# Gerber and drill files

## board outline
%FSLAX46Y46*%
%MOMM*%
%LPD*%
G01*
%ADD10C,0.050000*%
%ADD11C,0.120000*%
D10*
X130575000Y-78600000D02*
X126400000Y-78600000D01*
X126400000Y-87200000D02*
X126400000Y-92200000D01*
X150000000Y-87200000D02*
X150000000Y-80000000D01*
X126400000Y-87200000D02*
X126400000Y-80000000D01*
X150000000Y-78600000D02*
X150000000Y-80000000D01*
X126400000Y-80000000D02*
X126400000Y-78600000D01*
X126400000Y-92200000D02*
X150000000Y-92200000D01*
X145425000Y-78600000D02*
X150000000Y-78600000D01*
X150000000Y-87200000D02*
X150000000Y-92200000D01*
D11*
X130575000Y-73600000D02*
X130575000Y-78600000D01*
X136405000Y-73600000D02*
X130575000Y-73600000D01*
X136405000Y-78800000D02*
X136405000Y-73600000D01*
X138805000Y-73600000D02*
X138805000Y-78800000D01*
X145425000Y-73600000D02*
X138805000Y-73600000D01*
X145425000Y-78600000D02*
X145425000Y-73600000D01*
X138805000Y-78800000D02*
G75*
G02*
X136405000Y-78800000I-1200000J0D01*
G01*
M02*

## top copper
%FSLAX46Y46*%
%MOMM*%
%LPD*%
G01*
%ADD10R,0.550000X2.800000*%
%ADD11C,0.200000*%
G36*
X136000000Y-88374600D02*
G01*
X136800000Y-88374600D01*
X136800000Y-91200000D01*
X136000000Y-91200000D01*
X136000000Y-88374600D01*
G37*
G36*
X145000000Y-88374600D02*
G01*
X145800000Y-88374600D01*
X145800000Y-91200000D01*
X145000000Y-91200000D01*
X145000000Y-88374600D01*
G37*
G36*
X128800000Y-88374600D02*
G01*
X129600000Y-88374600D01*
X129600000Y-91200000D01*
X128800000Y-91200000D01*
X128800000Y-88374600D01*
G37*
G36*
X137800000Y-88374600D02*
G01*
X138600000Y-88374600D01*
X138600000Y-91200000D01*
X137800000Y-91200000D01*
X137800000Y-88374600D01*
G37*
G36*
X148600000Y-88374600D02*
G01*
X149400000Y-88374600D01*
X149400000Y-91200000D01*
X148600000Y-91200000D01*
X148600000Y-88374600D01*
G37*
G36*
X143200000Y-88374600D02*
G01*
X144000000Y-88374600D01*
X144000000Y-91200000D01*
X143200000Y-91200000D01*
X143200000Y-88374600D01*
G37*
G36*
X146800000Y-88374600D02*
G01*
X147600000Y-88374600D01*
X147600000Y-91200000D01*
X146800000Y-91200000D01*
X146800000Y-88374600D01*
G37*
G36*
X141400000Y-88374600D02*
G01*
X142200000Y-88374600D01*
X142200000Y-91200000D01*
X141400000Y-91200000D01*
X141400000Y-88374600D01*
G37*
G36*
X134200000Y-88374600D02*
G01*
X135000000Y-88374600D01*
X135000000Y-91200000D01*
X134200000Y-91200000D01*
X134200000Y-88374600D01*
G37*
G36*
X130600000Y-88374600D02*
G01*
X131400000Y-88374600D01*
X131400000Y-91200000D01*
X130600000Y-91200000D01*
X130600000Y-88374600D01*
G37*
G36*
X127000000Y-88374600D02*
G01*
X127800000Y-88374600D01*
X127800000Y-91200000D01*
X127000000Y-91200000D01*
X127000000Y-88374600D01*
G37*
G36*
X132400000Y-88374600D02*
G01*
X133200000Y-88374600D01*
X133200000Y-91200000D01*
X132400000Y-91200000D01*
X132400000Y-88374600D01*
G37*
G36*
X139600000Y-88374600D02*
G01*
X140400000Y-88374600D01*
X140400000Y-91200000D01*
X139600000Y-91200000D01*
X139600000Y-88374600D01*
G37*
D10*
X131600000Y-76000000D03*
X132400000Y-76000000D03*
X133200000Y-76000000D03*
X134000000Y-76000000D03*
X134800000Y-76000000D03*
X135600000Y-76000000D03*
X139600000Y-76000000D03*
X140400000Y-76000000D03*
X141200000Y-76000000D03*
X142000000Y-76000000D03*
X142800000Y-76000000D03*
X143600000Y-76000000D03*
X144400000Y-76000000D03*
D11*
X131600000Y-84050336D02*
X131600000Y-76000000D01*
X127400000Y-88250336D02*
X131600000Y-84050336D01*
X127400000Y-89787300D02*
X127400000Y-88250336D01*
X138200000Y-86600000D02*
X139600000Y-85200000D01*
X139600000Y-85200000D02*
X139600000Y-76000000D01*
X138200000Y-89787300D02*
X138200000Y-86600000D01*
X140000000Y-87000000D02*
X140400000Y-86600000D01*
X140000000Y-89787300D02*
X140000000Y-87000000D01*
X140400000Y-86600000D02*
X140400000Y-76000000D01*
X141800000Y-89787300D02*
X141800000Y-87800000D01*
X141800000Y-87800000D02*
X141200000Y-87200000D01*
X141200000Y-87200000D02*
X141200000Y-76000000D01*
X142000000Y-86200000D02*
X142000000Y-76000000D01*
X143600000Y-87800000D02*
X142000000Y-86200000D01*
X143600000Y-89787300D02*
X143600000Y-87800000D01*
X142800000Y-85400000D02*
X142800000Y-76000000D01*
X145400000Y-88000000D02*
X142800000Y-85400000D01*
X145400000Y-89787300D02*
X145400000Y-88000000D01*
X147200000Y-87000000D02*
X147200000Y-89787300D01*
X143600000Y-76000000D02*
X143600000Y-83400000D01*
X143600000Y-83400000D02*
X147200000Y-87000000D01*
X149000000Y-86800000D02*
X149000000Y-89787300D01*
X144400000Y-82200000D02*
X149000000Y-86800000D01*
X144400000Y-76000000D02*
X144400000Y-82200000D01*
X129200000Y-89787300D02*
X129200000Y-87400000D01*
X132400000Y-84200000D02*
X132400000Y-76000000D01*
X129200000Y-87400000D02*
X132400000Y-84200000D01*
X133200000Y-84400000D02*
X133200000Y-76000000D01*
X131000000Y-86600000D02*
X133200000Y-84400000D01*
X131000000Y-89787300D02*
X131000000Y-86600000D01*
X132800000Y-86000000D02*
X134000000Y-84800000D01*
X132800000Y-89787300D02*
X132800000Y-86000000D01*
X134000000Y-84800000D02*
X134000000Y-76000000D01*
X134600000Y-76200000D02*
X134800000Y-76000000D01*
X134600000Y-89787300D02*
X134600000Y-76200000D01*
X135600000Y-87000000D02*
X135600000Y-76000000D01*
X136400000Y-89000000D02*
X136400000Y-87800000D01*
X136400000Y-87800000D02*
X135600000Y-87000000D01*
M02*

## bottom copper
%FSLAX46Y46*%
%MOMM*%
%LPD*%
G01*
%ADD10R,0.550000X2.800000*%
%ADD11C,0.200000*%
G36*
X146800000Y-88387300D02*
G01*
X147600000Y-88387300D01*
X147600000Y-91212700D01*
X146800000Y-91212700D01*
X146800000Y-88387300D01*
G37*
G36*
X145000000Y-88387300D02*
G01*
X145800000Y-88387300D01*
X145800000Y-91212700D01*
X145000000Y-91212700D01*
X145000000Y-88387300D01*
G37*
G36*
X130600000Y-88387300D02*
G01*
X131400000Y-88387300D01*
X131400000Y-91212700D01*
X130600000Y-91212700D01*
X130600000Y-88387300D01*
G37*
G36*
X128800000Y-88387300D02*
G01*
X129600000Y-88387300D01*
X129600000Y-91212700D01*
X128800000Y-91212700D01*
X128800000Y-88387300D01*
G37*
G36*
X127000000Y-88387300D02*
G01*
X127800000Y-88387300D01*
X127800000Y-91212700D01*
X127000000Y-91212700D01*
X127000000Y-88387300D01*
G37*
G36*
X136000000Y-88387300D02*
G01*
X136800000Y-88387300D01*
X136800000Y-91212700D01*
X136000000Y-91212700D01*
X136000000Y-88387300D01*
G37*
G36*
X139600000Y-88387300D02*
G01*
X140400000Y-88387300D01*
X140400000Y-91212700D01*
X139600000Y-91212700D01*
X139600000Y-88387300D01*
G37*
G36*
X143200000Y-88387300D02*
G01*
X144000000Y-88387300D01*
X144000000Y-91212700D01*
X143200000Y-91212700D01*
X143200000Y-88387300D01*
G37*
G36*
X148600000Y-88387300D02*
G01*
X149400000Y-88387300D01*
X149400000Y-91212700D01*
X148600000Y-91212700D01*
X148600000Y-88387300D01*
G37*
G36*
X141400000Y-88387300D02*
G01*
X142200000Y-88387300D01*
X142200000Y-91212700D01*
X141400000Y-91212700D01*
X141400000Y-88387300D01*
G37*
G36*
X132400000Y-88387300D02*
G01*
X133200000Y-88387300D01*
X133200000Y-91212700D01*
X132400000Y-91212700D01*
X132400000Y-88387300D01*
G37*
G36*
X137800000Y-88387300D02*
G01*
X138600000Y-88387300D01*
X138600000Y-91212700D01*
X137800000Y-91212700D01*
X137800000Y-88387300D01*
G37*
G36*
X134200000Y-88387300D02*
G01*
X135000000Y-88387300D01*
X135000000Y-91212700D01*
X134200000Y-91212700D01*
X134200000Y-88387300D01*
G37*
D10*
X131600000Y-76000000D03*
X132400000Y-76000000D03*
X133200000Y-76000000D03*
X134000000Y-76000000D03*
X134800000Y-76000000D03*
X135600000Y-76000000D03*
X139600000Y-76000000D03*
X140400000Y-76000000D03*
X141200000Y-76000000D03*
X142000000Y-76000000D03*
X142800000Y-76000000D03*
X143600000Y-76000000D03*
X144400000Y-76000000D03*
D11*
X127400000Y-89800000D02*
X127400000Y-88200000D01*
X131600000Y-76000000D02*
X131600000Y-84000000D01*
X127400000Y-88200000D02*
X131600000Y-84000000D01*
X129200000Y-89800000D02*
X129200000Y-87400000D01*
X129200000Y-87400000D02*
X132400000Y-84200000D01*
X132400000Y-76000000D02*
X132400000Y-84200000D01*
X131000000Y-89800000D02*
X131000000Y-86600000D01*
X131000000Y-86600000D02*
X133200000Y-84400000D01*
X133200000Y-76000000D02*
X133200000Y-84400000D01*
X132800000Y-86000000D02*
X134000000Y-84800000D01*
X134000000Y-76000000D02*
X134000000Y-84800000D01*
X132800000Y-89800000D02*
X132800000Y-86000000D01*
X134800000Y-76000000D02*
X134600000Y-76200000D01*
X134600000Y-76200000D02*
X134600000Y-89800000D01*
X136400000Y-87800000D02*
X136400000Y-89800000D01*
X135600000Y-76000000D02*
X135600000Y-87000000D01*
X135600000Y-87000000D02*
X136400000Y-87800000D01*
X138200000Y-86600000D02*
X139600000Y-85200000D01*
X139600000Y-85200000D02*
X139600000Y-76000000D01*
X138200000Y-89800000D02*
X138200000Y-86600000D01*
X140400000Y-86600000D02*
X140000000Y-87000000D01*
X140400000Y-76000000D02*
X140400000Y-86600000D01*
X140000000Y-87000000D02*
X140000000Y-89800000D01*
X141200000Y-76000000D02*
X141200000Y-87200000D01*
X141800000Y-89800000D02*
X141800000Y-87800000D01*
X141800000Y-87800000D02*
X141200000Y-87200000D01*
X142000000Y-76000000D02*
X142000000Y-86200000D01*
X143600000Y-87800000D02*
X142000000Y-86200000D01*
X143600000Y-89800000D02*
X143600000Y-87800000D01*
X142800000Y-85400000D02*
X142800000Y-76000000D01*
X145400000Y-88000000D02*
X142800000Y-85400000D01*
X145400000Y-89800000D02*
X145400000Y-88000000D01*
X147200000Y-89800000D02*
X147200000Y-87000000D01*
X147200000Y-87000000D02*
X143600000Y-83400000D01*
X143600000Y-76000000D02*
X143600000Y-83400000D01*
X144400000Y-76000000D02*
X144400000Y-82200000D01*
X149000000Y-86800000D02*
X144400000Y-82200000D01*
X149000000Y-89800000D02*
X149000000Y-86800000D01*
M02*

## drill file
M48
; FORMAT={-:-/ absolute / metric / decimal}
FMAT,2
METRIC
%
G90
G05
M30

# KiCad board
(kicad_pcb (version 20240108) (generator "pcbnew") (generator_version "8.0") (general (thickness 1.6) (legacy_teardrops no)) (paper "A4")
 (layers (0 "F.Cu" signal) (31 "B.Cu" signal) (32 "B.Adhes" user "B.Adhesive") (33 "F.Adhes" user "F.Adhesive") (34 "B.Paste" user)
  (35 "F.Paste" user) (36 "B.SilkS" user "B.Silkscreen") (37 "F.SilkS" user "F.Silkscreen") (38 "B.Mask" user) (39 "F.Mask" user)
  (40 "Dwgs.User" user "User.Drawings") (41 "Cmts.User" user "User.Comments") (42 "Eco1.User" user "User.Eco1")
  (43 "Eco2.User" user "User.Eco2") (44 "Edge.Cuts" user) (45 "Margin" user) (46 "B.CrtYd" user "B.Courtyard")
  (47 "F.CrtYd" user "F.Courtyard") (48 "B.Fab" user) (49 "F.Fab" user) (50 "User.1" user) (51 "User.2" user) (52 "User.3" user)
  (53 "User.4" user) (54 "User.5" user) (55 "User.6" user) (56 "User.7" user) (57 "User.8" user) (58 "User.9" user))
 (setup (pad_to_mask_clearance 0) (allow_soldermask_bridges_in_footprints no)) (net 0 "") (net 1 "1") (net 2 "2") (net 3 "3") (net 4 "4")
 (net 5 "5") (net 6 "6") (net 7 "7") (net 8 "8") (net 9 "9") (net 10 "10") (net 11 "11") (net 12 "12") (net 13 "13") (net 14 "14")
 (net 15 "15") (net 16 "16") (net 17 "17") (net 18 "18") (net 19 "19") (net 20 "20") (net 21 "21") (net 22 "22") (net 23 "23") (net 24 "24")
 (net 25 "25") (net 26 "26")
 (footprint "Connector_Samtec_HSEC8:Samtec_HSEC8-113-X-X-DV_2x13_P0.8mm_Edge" (layer "B.Cu") (at 138 73.6)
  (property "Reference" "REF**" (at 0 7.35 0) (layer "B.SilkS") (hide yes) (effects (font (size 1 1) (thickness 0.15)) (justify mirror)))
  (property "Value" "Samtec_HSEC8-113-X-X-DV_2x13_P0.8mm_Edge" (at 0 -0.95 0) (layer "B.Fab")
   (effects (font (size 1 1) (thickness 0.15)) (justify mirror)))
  (fp_line (start -7.425 0) (end -7.425 5) (stroke (width 0.12) (type solid)) (layer "Edge.Cuts"))
  (fp_line (start -1.595 0) (end -7.425 0) (stroke (width 0.12) (type solid)) (layer "Edge.Cuts"))
  (fp_line (start -1.595 5.2) (end -1.595 0) (stroke (width 0.12) (type solid)) (layer "Edge.Cuts"))
  (fp_line (start 0.805 0) (end 0.805 5.2) (stroke (width 0.12) (type solid)) (layer "Edge.Cuts"))
  (fp_line (start 7.425 0) (end 0.805 0) (stroke (width 0.12) (type solid)) (layer "Edge.Cuts"))
  (fp_line (start 7.425 5) (end 7.425 0) (stroke (width 0.12) (type solid)) (layer "Edge.Cuts"))
  (fp_arc (start 0.805 5.2) (mid -0.395 6.4) (end -1.595 5.2) (stroke (width 0.12) (type solid)) (layer "Edge.Cuts"))
  (pad "1" connect rect (at -6.4 2.4) (size 0.55 2.8) (layers "B.Cu" "B.Mask") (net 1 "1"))
  (pad "2" connect rect (at -6.4 2.4) (size 0.55 2.8) (layers "F.Cu" "F.Mask") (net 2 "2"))
  (pad "3" connect rect (at -5.6 2.4) (size 0.55 2.8) (layers "B.Cu" "B.Mask") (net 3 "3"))
  (pad "4" connect rect (at -5.6 2.4) (size 0.55 2.8) (layers "F.Cu" "F.Mask") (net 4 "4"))
  (pad "5" connect rect (at -4.8 2.4) (size 0.55 2.8) (layers "B.Cu" "B.Mask") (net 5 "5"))
  (pad "6" connect rect (at -4.8 2.4) (size 0.55 2.8) (layers "F.Cu" "F.Mask") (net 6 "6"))
  (pad "7" connect rect (at -4 2.4) (size 0.55 2.8) (layers "B.Cu" "B.Mask") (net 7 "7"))
  (pad "8" connect rect (at -4 2.4) (size 0.55 2.8) (layers "F.Cu" "F.Mask") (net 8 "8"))
  (pad "9" connect rect (at -3.2 2.4) (size 0.55 2.8) (layers "B.Cu" "B.Mask") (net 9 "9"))
  (pad "10" connect rect (at -3.2 2.4) (size 0.55 2.8) (layers "F.Cu" "F.Mask") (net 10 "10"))
  (pad "11" connect rect (at -2.4 2.4) (size 0.55 2.8) (layers "B.Cu" "B.Mask") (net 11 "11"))
  (pad "12" connect rect (at -2.4 2.4) (size 0.55 2.8) (layers "F.Cu" "F.Mask") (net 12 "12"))
  (pad "13" connect rect (at 1.6 2.4) (size 0.55 2.8) (layers "B.Cu" "B.Mask") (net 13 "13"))
  (pad "14" connect rect (at 1.6 2.4) (size 0.55 2.8) (layers "F.Cu" "F.Mask") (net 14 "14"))
  (pad "15" connect rect (at 2.4 2.4) (size 0.55 2.8) (layers "B.Cu" "B.Mask") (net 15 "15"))
  (pad "16" connect rect (at 2.4 2.4) (size 0.55 2.8) (layers "F.Cu" "F.Mask") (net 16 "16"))
  (pad "17" connect rect (at 3.2 2.4) (size 0.55 2.8) (layers "B.Cu" "B.Mask") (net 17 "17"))
  (pad "18" connect rect (at 3.2 2.4) (size 0.55 2.8) (layers "F.Cu" "F.Mask") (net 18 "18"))
  (pad "19" connect rect (at 4 2.4) (size 0.55 2.8) (layers "B.Cu" "B.Mask") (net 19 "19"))
  (pad "20" connect rect (at 4 2.4) (size 0.55 2.8) (layers "F.Cu" "F.Mask") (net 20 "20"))
  (pad "21" connect rect (at 4.8 2.4) (size 0.55 2.8) (layers "B.Cu" "B.Mask") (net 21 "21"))
  (pad "22" connect rect (at 4.8 2.4) (size 0.55 2.8) (layers "F.Cu" "F.Mask") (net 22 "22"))
  (pad "23" connect rect (at 5.6 2.4) (size 0.55 2.8) (layers "B.Cu" "B.Mask") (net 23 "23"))
  (pad "24" connect rect (at 5.6 2.4) (size 0.55 2.8) (layers "F.Cu" "F.Mask") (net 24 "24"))
  (pad "25" connect rect (at 6.4 2.4) (size 0.55 2.8) (layers "B.Cu" "B.Mask") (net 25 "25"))
  (pad "26" connect rect (at 6.4 2.4) (size 0.55 2.8) (layers "F.Cu" "F.Mask") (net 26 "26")))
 (gr_rect (start 136 88.3746) (end 136.8 91.2) (stroke (width 0) (type solid)) (fill solid) (layer "F.Cu") (net 12))
 (gr_rect (start 145 88.3746) (end 145.8 91.2) (stroke (width 0) (type solid)) (fill solid) (layer "F.Cu") (net 22))
 (gr_rect (start 128.8 88.3746) (end 129.6 91.2) (stroke (width 0) (type solid)) (fill solid) (layer "F.Cu") (net 4))
 (gr_rect (start 137.8 88.3746) (end 138.6 91.2) (stroke (width 0) (type solid)) (fill solid) (layer "F.Cu") (net 14))
 (gr_rect (start 148.6 88.3746) (end 149.4 91.2) (stroke (width 0) (type solid)) (fill solid) (layer "F.Cu") (net 26))
 (gr_rect (start 143.2 88.3746) (end 144 91.2) (stroke (width 0) (type solid)) (fill solid) (layer "F.Cu") (net 20))
 (gr_rect (start 146.8 88.3746) (end 147.6 91.2) (stroke (width 0) (type solid)) (fill solid) (layer "F.Cu") (net 24))
 (gr_rect (start 141.4 88.3746) (end 142.2 91.2) (stroke (width 0) (type solid)) (fill solid) (layer "F.Cu") (net 18))
 (gr_rect (start 134.2 88.3746) (end 135 91.2) (stroke (width 0) (type solid)) (fill solid) (layer "F.Cu") (net 10))
 (gr_rect (start 130.6 88.3746) (end 131.4 91.2) (stroke (width 0) (type solid)) (fill solid) (layer "F.Cu") (net 6))
 (gr_rect (start 127 88.3746) (end 127.8 91.2) (stroke (width 0) (type solid)) (fill solid) (layer "F.Cu") (net 2))
 (gr_rect (start 132.4 88.3746) (end 133.2 91.2) (stroke (width 0) (type solid)) (fill solid) (layer "F.Cu") (net 8))
 (gr_rect (start 139.6 88.3746) (end 140.4 91.2) (stroke (width 0) (type solid)) (fill solid) (layer "F.Cu") (net 16))
 (gr_rect (start 146.8 88.3873) (end 147.6 91.2127) (stroke (width 0) (type solid)) (fill solid) (layer "B.Cu") (net 23))
 (gr_rect (start 145 88.3873) (end 145.8 91.2127) (stroke (width 0) (type solid)) (fill solid) (layer "B.Cu") (net 21))
 (gr_rect (start 130.6 88.3873) (end 131.4 91.2127) (stroke (width 0) (type solid)) (fill solid) (layer "B.Cu") (net 5))
 (gr_rect (start 128.8 88.3873) (end 129.6 91.2127) (stroke (width 0) (type solid)) (fill solid) (layer "B.Cu") (net 3))
 (gr_rect (start 127 88.3873) (end 127.8 91.2127) (stroke (width 0) (type solid)) (fill solid) (layer "B.Cu") (net 1))
 (gr_rect (start 136 88.3873) (end 136.8 91.2127) (stroke (width 0) (type solid)) (fill solid) (layer "B.Cu") (net 11))
 (gr_rect (start 139.6 88.3873) (end 140.4 91.2127) (stroke (width 0) (type solid)) (fill solid) (layer "B.Cu") (net 15))
 (gr_rect (start 143.2 88.3873) (end 144 91.2127) (stroke (width 0) (type solid)) (fill solid) (layer "B.Cu") (net 19))
 (gr_rect (start 148.6 88.3873) (end 149.4 91.2127) (stroke (width 0) (type solid)) (fill solid) (layer "B.Cu") (net 25))
 (gr_rect (start 141.4 88.3873) (end 142.2 91.2127) (stroke (width 0) (type solid)) (fill solid) (layer "B.Cu") (net 17))
 (gr_rect (start 132.4 88.3873) (end 133.2 91.2127) (stroke (width 0) (type solid)) (fill solid) (layer "B.Cu") (net 7))
 (gr_rect (start 137.8 88.3873) (end 138.6 91.2127) (stroke (width 0) (type solid)) (fill solid) (layer "B.Cu") (net 13))
 (gr_rect (start 134.2 88.3873) (end 135 91.2127) (stroke (width 0) (type solid)) (fill solid) (layer "B.Cu") (net 9))
 (gr_line (start 130.575 78.6) (end 126.4 78.6) (stroke (width 0.05) (type default)) (layer "Edge.Cuts"))
 (gr_line (start 126.4 87.2) (end 126.4 92.2) (stroke (width 0.05) (type default)) (layer "Edge.Cuts"))
 (gr_line (start 150 87.2) (end 150 80) (stroke (width 0.05) (type default)) (layer "Edge.Cuts"))
 (gr_line (start 126.4 87.2) (end 126.4 80) (stroke (width 0.05) (type default)) (layer "Edge.Cuts"))
 (gr_line (start 150 78.6) (end 150 80) (stroke (width 0.05) (type default)) (layer "Edge.Cuts"))
 (gr_line (start 126.4 80) (end 126.4 78.6) (stroke (width 0.05) (type default)) (layer "Edge.Cuts"))
 (gr_line (start 126.4 92.2) (end 150 92.2) (stroke (width 0.05) (type default)) (layer "Edge.Cuts"))
 (gr_line (start 145.425 78.6) (end 150 78.6) (stroke (width 0.05) (type default)) (layer "Edge.Cuts"))
 (gr_line (start 150 87.2) (end 150 92.2) (stroke (width 0.05) (type default)) (layer "Edge.Cuts"))
 (segment (start 131.6 84.050336) (end 131.6 76) (width 0.2) (layer "F.Cu") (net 2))
 (segment (start 127.4 88.250336) (end 131.6 84.050336) (width 0.2) (layer "F.Cu") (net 2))
 (segment (start 127.4 89.7873) (end 127.4 88.250336) (width 0.2) (layer "F.Cu") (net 2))
 (segment (start 127.4 89.8) (end 127.4 88.2) (width 0.2) (layer "B.Cu") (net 1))
 (segment (start 131.6 76) (end 131.6 84) (width 0.2) (layer "B.Cu") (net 1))
 (segment (start 127.4 88.2) (end 131.6 84) (width 0.2) (layer "B.Cu") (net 1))
 (segment (start 138.2 86.6) (end 139.6 85.2) (width 0.2) (layer "F.Cu") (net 14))
 (segment (start 139.6 85.2) (end 139.6 76) (width 0.2) (layer "F.Cu") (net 14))
 (segment (start 138.2 89.7873) (end 138.2 86.6) (width 0.2) (layer "F.Cu") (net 14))
 (segment (start 140 87) (end 140.4 86.6) (width 0.2) (layer "F.Cu") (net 16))
 (segment (start 140 89.7873) (end 140 87) (width 0.2) (layer "F.Cu") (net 16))
 (segment (start 140.4 86.6) (end 140.4 76) (width 0.2) (layer "F.Cu") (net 16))
 (segment (start 141.8 89.7873) (end 141.8 87.8) (width 0.2) (layer "F.Cu") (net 18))
 (segment (start 141.8 87.8) (end 141.2 87.2) (width 0.2) (layer "F.Cu") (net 18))
 (segment (start 141.2 87.2) (end 141.2 76) (width 0.2) (layer "F.Cu") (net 18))
 (segment (start 142 86.2) (end 142 76) (width 0.2) (layer "F.Cu") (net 20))
 (segment (start 143.6 87.8) (end 142 86.2) (width 0.2) (layer "F.Cu") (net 20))
 (segment (start 143.6 89.7873) (end 143.6 87.8) (width 0.2) (layer "F.Cu") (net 20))
 (segment (start 142.8 85.4) (end 142.8 76) (width 0.2) (layer "F.Cu") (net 22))
 (segment (start 145.4 88) (end 142.8 85.4) (width 0.2) (layer "F.Cu") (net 22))
 (segment (start 145.4 89.7873) (end 145.4 88) (width 0.2) (layer "F.Cu") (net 22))
 (segment (start 147.2 87) (end 147.2 89.7873) (width 0.2) (layer "F.Cu") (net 24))
 (segment (start 143.6 76) (end 143.6 83.4) (width 0.2) (layer "F.Cu") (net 24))
 (segment (start 143.6 83.4) (end 147.2 87) (width 0.2) (layer "F.Cu") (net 24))
 (segment (start 149 86.8) (end 149 89.7873) (width 0.2) (layer "F.Cu") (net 26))
 (segment (start 144.4 82.2) (end 149 86.8) (width 0.2) (layer "F.Cu") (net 26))
 (segment (start 144.4 76) (end 144.4 82.2) (width 0.2) (layer "F.Cu") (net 26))
 (segment (start 129.2 89.7873) (end 129.2 87.4) (width 0.2) (layer "F.Cu") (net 4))
 (segment (start 132.4 84.2) (end 132.4 76) (width 0.2) (layer "F.Cu") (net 4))
 (segment (start 129.2 87.4) (end 132.4 84.2) (width 0.2) (layer "F.Cu") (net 4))
 (segment (start 133.2 84.4) (end 133.2 76) (width 0.2) (layer "F.Cu") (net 6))
 (segment (start 131 86.6) (end 133.2 84.4) (width 0.2) (layer "F.Cu") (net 6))
 (segment (start 131 89.7873) (end 131 86.6) (width 0.2) (layer "F.Cu") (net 6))
 (segment (start 132.8 86) (end 134 84.8) (width 0.2) (layer "F.Cu") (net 8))
 (segment (start 132.8 89.7873) (end 132.8 86) (width 0.2) (layer "F.Cu") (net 8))
 (segment (start 134 84.8) (end 134 76) (width 0.2) (layer "F.Cu") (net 8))
 (segment (start 134.6 76.2) (end 134.8 76) (width 0.2) (layer "F.Cu") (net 10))
 (segment (start 134.6 89.7873) (end 134.6 76.2) (width 0.2) (layer "F.Cu") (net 10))
 (segment (start 135.6 87) (end 135.6 76) (width 0.2) (layer "F.Cu") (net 12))
 (segment (start 136.4 89) (end 136.4 87.8) (width 0.2) (layer "F.Cu") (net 12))
 (segment (start 136.4 87.8) (end 135.6 87) (width 0.2) (layer "F.Cu") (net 12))
 (segment (start 129.2 89.8) (end 129.2 87.4) (width 0.2) (layer "B.Cu") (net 3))
 (segment (start 129.2 87.4) (end 132.4 84.2) (width 0.2) (layer "B.Cu") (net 3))
 (segment (start 132.4 76) (end 132.4 84.2) (width 0.2) (layer "B.Cu") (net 3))
 (segment (start 131 89.8) (end 131 86.6) (width 0.2) (layer "B.Cu") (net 5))
 (segment (start 131 86.6) (end 133.2 84.4) (width 0.2) (layer "B.Cu") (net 5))
 (segment (start 133.2 76) (end 133.2 84.4) (width 0.2) (layer "B.Cu") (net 5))
 (segment (start 132.8 86) (end 134 84.8) (width 0.2) (layer "B.Cu") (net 7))
 (segment (start 134 76) (end 134 84.8) (width 0.2) (layer "B.Cu") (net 7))
 (segment (start 132.8 89.8) (end 132.8 86) (width 0.2) (layer "B.Cu") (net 7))
 (segment (start 134.8 76) (end 134.6 76.2) (width 0.2) (layer "B.Cu") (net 9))
 (segment (start 134.6 76.2) (end 134.6 89.8) (width 0.2) (layer "B.Cu") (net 9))
 (segment (start 136.4 87.8) (end 136.4 89.8) (width 0.2) (layer "B.Cu") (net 11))
 (segment (start 135.6 76) (end 135.6 87) (width 0.2) (layer "B.Cu") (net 11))
 (segment (start 135.6 87) (end 136.4 87.8) (width 0.2) (layer "B.Cu") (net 11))
 (segment (start 138.2 86.6) (end 139.6 85.2) (width 0.2) (layer "B.Cu") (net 13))
 (segment (start 139.6 85.2) (end 139.6 76) (width 0.2) (layer "B.Cu") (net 13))
 (segment (start 138.2 89.8) (end 138.2 86.6) (width 0.2) (layer "B.Cu") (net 13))
 (segment (start 140.4 86.6) (end 140 87) (width 0.2) (layer "B.Cu") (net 15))
 (segment (start 140.4 76) (end 140.4 86.6) (width 0.2) (layer "B.Cu") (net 15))
 (segment (start 140 87) (end 140 89.8) (width 0.2) (layer "B.Cu") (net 15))
 (segment (start 141.2 76) (end 141.2 87.2) (width 0.2) (layer "B.Cu") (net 17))
 (segment (start 141.8 89.8) (end 141.8 87.8) (width 0.2) (layer "B.Cu") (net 17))
 (segment (start 141.8 87.8) (end 141.2 87.2) (width 0.2) (layer "B.Cu") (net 17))
 (segment (start 142 76) (end 142 86.2) (width 0.2) (layer "B.Cu") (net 19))
 (segment (start 143.6 87.8) (end 142 86.2) (width 0.2) (layer "B.Cu") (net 19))
 (segment (start 143.6 89.8) (end 143.6 87.8) (width 0.2) (layer "B.Cu") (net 19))
 (segment (start 142.8 85.4) (end 142.8 76) (width 0.2) (layer "B.Cu") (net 21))
 (segment (start 145.4 88) (end 142.8 85.4) (width 0.2) (layer "B.Cu") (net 21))
 (segment (start 145.4 89.8) (end 145.4 88) (width 0.2) (layer "B.Cu") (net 21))
 (segment (start 147.2 89.8) (end 147.2 87) (width 0.2) (layer "B.Cu") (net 23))
 (segment (start 147.2 87) (end 143.6 83.4) (width 0.2) (layer "B.Cu") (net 23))
 (segment (start 143.6 76) (end 143.6 83.4) (width 0.2) (layer "B.Cu") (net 23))
 (segment (start 144.4 76) (end 144.4 82.2) (width 0.2) (layer "B.Cu") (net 25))
 (segment (start 149 86.8) (end 144.4 82.2) (width 0.2) (layer "B.Cu") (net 25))
 (segment (start 149 89.8) (end 149 86.8) (width 0.2) (layer "B.Cu") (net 25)))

